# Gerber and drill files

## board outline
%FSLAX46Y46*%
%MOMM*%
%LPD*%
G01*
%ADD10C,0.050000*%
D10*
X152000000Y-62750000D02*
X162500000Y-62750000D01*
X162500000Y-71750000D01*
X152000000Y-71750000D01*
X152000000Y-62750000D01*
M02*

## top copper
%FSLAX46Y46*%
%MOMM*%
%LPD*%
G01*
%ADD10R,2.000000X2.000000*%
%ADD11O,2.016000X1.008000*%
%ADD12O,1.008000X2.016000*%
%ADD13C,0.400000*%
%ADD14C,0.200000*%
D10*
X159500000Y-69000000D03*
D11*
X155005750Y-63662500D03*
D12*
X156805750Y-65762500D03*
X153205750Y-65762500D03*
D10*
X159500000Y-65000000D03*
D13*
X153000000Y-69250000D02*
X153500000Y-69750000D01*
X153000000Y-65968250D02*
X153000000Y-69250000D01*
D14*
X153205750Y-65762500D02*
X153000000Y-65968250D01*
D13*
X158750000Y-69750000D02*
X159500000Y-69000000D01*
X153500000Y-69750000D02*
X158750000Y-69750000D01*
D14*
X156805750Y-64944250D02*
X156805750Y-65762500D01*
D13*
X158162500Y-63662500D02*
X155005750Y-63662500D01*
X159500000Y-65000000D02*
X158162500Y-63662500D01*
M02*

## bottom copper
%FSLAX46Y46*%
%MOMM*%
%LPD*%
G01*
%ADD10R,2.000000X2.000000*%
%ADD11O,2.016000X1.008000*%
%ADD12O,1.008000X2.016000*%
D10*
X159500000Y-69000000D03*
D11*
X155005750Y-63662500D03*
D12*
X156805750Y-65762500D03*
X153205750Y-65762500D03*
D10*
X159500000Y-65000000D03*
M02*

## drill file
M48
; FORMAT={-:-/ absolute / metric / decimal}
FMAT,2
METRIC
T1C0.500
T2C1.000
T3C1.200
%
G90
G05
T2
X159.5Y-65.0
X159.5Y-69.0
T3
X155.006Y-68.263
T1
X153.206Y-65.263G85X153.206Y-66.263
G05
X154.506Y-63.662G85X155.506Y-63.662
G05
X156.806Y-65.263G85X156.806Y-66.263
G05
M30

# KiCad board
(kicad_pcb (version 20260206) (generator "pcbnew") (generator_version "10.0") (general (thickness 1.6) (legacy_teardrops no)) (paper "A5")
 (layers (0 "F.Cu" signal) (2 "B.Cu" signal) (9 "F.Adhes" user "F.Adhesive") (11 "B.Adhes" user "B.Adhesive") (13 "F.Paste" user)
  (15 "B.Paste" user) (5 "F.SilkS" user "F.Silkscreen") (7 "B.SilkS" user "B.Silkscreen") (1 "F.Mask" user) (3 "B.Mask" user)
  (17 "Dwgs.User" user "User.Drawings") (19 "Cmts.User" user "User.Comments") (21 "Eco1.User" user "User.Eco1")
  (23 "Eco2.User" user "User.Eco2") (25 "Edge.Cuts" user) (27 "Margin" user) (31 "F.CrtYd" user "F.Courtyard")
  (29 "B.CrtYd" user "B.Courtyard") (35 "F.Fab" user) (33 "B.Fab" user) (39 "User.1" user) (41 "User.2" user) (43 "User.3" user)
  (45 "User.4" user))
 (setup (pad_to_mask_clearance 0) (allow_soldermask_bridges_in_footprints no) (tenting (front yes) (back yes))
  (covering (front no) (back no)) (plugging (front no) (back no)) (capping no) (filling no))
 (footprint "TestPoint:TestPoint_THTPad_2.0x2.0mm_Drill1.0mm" (layer "F.Cu") (at 159.5 69)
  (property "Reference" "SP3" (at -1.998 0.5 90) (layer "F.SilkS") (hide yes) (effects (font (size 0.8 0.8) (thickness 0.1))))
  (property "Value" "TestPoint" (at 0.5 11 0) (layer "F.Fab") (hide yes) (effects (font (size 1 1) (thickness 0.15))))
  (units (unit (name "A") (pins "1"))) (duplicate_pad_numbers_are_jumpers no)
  (pad "1" thru_hole rect (at 0 0) (size 2 2) (drill 1) (layers "*.Cu" "*.Mask") (remove_unused_layers no) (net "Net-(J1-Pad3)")))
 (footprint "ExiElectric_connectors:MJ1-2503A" (layer "F.Cu") (at 155.00575 68.2625)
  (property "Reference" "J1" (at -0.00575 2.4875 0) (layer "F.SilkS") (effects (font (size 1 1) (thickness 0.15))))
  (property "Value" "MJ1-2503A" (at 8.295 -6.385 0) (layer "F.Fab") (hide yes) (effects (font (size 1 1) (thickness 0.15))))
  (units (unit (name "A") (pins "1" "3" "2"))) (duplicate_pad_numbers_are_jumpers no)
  (pad "" np_thru_hole circle (at 0 0) (size 1.2 1.2) (drill 1.2) (layers "*.Cu" "*.Mask"))
  (pad "1" thru_hole oval (at 0 -4.6) (size 2.016 1.008) (drill oval 1.5 0.5) (layers "*.Cu" "*.Mask") (remove_unused_layers no)
   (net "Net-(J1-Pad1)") (solder_mask_margin 0.102))
  (pad "2" thru_hole oval (at 1.8 -2.5) (size 1.008 2.016) (drill oval 0.5 1.5) (layers "*.Cu" "*.Mask") (remove_unused_layers no)
   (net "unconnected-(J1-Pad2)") (solder_mask_margin 0.102))
  (pad "3" thru_hole oval (at -1.8 -2.5) (size 1.008 2.016) (drill oval 0.5 1.5) (layers "*.Cu" "*.Mask") (remove_unused_layers no)
   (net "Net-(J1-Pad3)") (solder_mask_margin 0.102)))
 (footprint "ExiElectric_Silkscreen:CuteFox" (layer "F.Cu") (at 155 66)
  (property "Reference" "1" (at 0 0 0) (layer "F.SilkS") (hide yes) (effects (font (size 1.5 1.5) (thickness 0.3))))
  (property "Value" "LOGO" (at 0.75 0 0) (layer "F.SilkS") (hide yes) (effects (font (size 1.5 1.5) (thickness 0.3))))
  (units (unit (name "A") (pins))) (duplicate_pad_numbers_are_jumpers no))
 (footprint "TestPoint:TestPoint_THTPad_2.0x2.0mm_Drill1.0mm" (layer "F.Cu") (at 159.5 65)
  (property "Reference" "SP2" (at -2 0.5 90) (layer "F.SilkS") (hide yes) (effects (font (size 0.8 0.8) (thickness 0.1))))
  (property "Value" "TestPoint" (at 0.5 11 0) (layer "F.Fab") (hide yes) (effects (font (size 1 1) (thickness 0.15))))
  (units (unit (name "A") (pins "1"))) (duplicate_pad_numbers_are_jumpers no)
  (pad "1" thru_hole rect (at 0 0) (size 2 2) (drill 1) (layers "*.Cu" "*.Mask") (remove_unused_layers no) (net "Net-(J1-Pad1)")))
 (gr_rect (start 152 62.75) (end 162.5 71.75) (stroke (width 0.05) (type default)) (fill no) (layer "Edge.Cuts"))
 (segment (start 153 69.25) (end 153.5 69.75) (width 0.4) (layer "F.Cu") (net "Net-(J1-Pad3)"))
 (segment (start 153 65.96825) (end 153 69.25) (width 0.4) (layer "F.Cu") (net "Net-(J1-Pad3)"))
 (segment (start 153.20575 65.7625) (end 153 65.96825) (width 0.2) (layer "F.Cu") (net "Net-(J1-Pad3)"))
 (segment (start 158.75 69.75) (end 159.5 69) (width 0.4) (layer "F.Cu") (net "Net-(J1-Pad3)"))
 (segment (start 153.5 69.75) (end 158.75 69.75) (width 0.4) (layer "F.Cu") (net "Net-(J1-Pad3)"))
 (segment (start 156.80575 64.94425) (end 156.80575 65.7625) (width 0.2) (layer "F.Cu") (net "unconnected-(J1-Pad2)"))
 (segment (start 158.1625 63.6625) (end 155.00575 63.6625) (width 0.4) (layer "F.Cu") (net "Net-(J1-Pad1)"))
 (segment (start 159.5 65) (end 158.1625 63.6625) (width 0.4) (layer "F.Cu") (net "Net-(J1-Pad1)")))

